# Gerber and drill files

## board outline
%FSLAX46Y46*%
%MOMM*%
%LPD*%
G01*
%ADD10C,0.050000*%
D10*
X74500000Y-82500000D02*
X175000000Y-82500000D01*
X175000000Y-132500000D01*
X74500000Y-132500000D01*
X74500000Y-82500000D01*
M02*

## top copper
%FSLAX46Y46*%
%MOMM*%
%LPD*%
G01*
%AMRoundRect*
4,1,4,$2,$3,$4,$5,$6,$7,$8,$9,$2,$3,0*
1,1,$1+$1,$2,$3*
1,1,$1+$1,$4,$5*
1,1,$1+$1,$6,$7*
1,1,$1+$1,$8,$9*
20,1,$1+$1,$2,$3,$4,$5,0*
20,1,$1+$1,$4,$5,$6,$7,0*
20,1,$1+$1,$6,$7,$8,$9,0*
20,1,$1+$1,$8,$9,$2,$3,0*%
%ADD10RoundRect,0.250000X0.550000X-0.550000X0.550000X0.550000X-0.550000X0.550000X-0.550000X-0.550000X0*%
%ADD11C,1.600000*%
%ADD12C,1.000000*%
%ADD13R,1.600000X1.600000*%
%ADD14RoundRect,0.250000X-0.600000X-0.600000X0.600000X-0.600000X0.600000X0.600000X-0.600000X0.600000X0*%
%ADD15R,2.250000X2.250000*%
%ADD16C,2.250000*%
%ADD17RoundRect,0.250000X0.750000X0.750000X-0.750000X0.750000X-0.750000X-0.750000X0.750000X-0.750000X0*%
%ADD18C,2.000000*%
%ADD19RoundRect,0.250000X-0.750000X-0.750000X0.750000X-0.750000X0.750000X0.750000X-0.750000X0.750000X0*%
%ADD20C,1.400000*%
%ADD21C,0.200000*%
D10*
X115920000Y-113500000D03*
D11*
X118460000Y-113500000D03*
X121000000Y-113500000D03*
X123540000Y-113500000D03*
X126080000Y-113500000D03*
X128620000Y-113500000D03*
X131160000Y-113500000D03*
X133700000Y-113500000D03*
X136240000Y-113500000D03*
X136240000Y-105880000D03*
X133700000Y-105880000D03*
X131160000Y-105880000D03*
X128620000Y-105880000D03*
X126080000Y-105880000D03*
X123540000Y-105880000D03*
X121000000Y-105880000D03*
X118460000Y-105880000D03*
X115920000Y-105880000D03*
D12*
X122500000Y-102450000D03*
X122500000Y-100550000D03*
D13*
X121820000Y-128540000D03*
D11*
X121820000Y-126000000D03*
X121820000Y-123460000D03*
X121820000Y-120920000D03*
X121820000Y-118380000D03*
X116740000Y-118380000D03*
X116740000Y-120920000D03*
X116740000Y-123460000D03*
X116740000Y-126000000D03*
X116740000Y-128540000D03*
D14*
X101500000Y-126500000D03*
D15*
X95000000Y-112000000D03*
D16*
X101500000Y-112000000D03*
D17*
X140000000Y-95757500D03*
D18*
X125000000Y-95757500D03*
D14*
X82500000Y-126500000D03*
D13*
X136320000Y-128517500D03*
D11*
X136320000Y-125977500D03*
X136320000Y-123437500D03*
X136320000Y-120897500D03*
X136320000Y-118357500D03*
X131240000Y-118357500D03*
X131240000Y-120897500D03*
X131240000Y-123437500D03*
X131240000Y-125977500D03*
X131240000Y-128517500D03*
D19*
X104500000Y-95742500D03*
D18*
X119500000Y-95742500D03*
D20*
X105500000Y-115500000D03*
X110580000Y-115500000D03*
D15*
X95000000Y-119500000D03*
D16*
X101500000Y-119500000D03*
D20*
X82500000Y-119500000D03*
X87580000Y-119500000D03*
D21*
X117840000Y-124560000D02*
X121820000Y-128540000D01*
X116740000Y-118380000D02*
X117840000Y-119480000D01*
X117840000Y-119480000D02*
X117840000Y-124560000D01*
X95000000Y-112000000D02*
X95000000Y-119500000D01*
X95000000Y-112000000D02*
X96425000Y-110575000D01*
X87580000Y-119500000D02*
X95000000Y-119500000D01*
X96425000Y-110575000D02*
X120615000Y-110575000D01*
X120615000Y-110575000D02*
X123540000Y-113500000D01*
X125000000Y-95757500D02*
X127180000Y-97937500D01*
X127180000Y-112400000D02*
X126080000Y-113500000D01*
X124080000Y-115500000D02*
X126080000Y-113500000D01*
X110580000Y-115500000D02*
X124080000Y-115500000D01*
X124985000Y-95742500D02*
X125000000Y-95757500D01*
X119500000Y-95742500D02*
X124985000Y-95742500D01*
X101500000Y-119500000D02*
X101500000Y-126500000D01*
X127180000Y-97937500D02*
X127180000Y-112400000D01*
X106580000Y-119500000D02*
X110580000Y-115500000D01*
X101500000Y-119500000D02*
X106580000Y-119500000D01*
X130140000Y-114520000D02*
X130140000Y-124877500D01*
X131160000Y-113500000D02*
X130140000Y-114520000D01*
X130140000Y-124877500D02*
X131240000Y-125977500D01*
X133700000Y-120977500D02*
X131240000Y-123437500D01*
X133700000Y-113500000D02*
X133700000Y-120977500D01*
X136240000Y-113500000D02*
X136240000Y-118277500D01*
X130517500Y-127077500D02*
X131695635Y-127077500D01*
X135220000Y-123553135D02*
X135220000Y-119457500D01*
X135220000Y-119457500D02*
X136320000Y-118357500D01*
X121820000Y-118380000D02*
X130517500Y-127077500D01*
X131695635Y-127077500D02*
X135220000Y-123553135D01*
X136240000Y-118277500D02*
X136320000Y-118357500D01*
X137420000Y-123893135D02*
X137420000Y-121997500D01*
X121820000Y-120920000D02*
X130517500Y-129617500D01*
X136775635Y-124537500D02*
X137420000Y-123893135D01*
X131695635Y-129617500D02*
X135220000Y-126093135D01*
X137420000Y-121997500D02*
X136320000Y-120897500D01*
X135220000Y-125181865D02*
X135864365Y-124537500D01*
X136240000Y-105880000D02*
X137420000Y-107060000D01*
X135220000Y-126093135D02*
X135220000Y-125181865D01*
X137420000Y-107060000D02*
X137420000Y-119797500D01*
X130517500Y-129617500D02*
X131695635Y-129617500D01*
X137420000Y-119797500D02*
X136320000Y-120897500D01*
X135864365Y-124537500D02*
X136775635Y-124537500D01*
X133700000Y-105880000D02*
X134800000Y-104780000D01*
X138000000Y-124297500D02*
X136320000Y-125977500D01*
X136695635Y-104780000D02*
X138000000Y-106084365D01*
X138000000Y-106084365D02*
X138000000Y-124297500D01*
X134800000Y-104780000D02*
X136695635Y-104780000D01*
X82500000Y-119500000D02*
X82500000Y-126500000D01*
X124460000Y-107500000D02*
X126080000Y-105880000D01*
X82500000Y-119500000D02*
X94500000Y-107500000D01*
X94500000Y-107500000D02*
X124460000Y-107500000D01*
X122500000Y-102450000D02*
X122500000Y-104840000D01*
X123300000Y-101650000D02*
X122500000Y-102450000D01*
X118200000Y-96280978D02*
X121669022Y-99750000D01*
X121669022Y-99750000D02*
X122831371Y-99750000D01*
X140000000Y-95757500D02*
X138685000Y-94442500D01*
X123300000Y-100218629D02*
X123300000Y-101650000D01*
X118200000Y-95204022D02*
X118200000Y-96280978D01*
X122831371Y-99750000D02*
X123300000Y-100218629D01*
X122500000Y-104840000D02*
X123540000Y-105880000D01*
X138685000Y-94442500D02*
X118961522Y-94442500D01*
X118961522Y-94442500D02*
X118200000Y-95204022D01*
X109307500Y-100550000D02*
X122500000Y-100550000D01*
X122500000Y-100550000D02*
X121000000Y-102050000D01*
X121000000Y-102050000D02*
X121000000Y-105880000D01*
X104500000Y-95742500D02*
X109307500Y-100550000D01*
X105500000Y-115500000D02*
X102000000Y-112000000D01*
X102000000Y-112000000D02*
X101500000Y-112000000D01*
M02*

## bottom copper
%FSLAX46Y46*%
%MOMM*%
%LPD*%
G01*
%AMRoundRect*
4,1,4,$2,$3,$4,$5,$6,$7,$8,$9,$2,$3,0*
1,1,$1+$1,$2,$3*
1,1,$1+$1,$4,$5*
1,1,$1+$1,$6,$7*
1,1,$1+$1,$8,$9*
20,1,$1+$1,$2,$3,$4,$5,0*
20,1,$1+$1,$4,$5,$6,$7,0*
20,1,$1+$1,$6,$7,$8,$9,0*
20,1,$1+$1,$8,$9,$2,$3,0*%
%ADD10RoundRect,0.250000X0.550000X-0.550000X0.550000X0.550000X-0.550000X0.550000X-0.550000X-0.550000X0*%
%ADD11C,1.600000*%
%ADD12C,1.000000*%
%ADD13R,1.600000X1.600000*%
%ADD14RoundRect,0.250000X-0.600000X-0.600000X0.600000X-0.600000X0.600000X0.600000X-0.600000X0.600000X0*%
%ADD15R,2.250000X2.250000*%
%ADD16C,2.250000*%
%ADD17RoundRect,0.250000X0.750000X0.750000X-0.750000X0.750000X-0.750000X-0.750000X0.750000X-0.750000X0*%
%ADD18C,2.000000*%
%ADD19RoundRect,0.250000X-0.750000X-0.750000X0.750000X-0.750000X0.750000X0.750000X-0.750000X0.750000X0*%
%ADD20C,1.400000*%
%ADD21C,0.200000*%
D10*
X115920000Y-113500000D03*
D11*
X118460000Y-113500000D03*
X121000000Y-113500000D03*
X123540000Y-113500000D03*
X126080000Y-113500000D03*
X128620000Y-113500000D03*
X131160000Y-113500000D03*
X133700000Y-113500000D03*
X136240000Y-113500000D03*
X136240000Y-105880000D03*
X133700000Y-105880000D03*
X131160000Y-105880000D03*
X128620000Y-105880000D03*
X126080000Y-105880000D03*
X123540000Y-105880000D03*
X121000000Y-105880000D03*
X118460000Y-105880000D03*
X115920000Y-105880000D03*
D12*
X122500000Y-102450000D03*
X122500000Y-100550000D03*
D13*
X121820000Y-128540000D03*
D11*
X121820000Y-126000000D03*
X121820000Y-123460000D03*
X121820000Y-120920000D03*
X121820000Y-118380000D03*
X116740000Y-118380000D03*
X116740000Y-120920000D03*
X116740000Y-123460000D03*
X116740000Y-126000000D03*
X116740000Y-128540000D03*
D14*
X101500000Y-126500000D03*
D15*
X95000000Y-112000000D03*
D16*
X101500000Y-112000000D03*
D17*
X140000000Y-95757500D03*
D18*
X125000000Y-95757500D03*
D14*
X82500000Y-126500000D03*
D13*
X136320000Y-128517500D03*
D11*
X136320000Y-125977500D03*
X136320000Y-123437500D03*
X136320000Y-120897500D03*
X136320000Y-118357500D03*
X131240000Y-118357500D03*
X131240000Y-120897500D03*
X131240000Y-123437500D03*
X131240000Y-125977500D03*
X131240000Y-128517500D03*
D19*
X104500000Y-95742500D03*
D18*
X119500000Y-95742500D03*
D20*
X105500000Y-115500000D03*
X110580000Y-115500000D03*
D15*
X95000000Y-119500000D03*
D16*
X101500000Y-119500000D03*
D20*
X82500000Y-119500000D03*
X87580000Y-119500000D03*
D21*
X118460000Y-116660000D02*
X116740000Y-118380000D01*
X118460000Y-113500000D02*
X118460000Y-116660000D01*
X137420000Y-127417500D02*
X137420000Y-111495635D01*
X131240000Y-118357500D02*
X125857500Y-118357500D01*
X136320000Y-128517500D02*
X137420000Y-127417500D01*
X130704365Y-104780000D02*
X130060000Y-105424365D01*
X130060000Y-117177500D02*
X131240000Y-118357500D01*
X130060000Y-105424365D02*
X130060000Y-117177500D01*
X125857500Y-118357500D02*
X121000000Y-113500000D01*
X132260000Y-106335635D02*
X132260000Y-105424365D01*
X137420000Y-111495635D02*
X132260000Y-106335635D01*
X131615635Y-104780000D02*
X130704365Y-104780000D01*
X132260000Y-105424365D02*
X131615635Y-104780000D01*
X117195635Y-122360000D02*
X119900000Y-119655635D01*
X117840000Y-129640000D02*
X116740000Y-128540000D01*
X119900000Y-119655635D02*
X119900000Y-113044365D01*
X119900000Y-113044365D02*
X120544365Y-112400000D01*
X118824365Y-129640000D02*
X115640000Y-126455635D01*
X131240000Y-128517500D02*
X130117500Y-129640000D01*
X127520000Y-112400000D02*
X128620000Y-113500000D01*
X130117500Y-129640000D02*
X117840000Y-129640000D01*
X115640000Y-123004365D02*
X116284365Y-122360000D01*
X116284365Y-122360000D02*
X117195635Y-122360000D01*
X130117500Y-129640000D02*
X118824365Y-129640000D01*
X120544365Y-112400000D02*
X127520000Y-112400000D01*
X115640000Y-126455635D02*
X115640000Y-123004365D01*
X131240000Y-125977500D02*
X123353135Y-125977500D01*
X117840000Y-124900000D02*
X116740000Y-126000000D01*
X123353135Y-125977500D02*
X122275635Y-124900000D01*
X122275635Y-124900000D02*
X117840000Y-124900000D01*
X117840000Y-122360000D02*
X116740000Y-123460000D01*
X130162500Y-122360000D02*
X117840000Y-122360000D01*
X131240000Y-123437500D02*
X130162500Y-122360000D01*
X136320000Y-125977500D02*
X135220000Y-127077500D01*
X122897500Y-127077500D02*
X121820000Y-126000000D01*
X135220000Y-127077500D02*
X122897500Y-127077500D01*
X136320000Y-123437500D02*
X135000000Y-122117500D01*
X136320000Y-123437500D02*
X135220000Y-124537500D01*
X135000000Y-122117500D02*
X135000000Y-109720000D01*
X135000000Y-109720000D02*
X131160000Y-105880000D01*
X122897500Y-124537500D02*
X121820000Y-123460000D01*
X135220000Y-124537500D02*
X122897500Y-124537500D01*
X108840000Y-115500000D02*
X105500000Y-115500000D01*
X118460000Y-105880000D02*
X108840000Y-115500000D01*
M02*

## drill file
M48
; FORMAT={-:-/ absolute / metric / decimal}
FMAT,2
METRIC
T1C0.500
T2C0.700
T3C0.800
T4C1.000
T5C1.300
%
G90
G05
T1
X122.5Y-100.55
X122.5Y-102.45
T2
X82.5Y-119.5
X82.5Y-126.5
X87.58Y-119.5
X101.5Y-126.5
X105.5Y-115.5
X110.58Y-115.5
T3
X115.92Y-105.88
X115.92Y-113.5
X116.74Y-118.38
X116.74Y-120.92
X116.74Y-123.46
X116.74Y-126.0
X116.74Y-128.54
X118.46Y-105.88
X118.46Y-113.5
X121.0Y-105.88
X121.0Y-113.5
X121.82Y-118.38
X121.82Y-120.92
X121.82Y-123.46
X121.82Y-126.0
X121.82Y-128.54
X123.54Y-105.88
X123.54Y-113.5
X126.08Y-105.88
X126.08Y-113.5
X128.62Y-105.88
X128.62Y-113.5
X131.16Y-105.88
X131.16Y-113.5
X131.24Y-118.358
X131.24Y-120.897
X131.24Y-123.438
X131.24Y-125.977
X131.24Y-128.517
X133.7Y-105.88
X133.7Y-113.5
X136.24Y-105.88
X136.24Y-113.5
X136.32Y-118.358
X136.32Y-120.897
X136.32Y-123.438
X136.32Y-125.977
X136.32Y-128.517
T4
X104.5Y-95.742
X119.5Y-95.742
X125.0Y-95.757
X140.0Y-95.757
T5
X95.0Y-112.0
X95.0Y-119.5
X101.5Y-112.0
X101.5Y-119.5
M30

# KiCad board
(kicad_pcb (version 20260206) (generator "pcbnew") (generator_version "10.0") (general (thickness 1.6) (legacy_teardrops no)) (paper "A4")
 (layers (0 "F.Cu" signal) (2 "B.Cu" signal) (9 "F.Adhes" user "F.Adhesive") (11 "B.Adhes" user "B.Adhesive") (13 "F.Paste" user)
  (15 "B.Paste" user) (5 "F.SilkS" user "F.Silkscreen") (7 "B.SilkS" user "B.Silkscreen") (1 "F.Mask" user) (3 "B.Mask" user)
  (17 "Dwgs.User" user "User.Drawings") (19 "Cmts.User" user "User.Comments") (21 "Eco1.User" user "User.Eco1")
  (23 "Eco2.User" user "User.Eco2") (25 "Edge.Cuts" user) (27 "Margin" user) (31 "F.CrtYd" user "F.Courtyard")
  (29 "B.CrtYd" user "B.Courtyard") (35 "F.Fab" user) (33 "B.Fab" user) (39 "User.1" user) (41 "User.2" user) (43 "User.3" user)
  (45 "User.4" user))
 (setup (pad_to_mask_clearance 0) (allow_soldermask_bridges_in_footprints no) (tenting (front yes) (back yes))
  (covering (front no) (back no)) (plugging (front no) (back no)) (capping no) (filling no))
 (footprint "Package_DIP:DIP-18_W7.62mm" (layer "F.Cu") (at 115.92 113.5 90)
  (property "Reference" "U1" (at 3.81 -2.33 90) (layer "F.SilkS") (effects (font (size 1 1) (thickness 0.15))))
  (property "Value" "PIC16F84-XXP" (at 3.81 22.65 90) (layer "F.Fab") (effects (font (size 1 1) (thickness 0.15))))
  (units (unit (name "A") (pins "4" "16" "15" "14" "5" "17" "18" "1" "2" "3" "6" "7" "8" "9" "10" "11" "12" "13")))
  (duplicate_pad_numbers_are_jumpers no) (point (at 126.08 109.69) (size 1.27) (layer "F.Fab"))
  (pad "1" thru_hole roundrect (at 0 0 90) (size 1.6 1.6) (drill 0.8) (layers "*.Cu" "*.Mask") (remove_unused_layers no)
   (roundrect_rratio 0.15625) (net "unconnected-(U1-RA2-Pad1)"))
  (pad "2" thru_hole circle (at 0 2.54 90) (size 1.6 1.6) (drill 0.8) (layers "*.Cu" "*.Mask") (remove_unused_layers no)
   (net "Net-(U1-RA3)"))
  (pad "3" thru_hole circle (at 0 5.08 90) (size 1.6 1.6) (drill 0.8) (layers "*.Cu" "*.Mask") (remove_unused_layers no)
   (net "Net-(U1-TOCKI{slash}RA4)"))
  (pad "4" thru_hole circle (at 0 7.62 90) (size 1.6 1.6) (drill 0.8) (layers "*.Cu" "*.Mask") (remove_unused_layers no)
   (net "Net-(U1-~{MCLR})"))
  (pad "5" thru_hole circle (at 0 10.16 90) (size 1.6 1.6) (drill 0.8) (layers "*.Cu" "*.Mask") (remove_unused_layers no) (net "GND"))
  (pad "6" thru_hole circle (at 0 12.7 90) (size 1.6 1.6) (drill 0.8) (layers "*.Cu" "*.Mask") (remove_unused_layers no)
   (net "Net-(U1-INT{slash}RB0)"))
  (pad "7" thru_hole circle (at 0 15.24 90) (size 1.6 1.6) (drill 0.8) (layers "*.Cu" "*.Mask") (remove_unused_layers no)
   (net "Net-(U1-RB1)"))
  (pad "8" thru_hole circle (at 0 17.78 90) (size 1.6 1.6) (drill 0.8) (layers "*.Cu" "*.Mask") (remove_unused_layers no)
   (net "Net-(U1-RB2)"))
  (pad "9" thru_hole circle (at 0 20.32 90) (size 1.6 1.6) (drill 0.8) (layers "*.Cu" "*.Mask") (remove_unused_layers no)
   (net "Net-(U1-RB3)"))
  (pad "10" thru_hole circle (at 7.62 20.32 90) (size 1.6 1.6) (drill 0.8) (layers "*.Cu" "*.Mask") (remove_unused_layers no)
   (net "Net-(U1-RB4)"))
  (pad "11" thru_hole circle (at 7.62 17.78 90) (size 1.6 1.6) (drill 0.8) (layers "*.Cu" "*.Mask") (remove_unused_layers no)
   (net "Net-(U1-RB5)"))
  (pad "12" thru_hole circle (at 7.62 15.24 90) (size 1.6 1.6) (drill 0.8) (layers "*.Cu" "*.Mask") (remove_unused_layers no)
   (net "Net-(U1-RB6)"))
  (pad "13" thru_hole circle (at 7.62 12.7 90) (size 1.6 1.6) (drill 0.8) (layers "*.Cu" "*.Mask") (remove_unused_layers no)
   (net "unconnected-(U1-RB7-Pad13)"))
  (pad "14" thru_hole circle (at 7.62 10.16 90) (size 1.6 1.6) (drill 0.8) (layers "*.Cu" "*.Mask") (remove_unused_layers no) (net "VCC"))
  (pad "15" thru_hole circle (at 7.62 7.62 90) (size 1.6 1.6) (drill 0.8) (layers "*.Cu" "*.Mask") (remove_unused_layers no)
   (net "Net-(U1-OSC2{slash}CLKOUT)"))
  (pad "16" thru_hole circle (at 7.62 5.08 90) (size 1.6 1.6) (drill 0.8) (layers "*.Cu" "*.Mask") (remove_unused_layers no)
   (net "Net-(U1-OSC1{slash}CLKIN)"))
  (pad "17" thru_hole circle (at 7.62 2.54 90) (size 1.6 1.6) (drill 0.8) (layers "*.Cu" "*.Mask") (remove_unused_layers no)
   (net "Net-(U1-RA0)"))
  (pad "18" thru_hole circle (at 7.62 0 90) (size 1.6 1.6) (drill 0.8) (layers "*.Cu" "*.Mask") (remove_unused_layers no)
   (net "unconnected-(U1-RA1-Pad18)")))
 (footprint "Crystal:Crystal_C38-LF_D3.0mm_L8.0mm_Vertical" (layer "F.Cu") (at 122.5 102.45 90)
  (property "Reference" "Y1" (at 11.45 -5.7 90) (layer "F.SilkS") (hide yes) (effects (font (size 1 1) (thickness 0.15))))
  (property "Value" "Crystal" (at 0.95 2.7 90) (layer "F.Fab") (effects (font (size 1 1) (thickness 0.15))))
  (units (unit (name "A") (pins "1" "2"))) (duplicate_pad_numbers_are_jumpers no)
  (pad "1" thru_hole circle (at 0 0 90) (size 1 1) (drill 0.5) (layers "*.Cu" "*.Mask") (remove_unused_layers no)
   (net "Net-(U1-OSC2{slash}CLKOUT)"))
  (pad "2" thru_hole circle (at 1.9 0 90) (size 1 1) (drill 0.5) (layers "*.Cu" "*.Mask") (remove_unused_layers no)
   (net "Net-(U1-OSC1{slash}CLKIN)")))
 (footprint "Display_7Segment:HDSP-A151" (layer "F.Cu") (at 121.82 128.54 180)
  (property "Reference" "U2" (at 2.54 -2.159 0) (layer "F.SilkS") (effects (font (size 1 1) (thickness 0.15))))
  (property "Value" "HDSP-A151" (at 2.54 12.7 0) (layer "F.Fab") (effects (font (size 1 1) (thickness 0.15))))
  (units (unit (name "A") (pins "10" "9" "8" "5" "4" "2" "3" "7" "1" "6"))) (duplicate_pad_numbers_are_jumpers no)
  (pad "1" thru_hole rect (at 0 0 180) (size 1.6 1.6) (drill 0.8) (layers "*.Cu" "*.Mask") (remove_unused_layers no) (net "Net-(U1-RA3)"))
  (pad "2" thru_hole circle (at 0 2.54 180) (size 1.6 1.6) (drill 0.8) (layers "*.Cu" "*.Mask") (remove_unused_layers no)
   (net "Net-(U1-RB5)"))
  (pad "3" thru_hole circle (at 0 5.08 180) (size 1.6 1.6) (drill 0.8) (layers "*.Cu" "*.Mask") (remove_unused_layers no)
   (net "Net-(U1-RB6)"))
  (pad "4" thru_hole circle (at 0 7.62 180) (size 1.6 1.6) (drill 0.8) (layers "*.Cu" "*.Mask") (remove_unused_layers no)
   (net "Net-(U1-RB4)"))
  (pad "5" thru_hole circle (at 0 10.16 180) (size 1.6 1.6) (drill 0.8) (layers "*.Cu" "*.Mask") (remove_unused_layers no)
   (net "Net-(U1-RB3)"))
  (pad "6" thru_hole circle (at 5.08 10.16 180) (size 1.6 1.6) (drill 0.8) (layers "*.Cu" "*.Mask") (remove_unused_layers no)
   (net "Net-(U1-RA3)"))
  (pad "7" thru_hole circle (at 5.08 7.62 180) (size 1.6 1.6) (drill 0.8) (layers "*.Cu" "*.Mask") (remove_unused_layers no)
   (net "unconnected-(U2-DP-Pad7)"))
  (pad "8" thru_hole circle (at 5.08 5.08 180) (size 1.6 1.6) (drill 0.8) (layers "*.Cu" "*.Mask") (remove_unused_layers no)
   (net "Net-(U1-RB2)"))
  (pad "9" thru_hole circle (at 5.08 2.54 180) (size 1.6 1.6) (drill 0.8) (layers "*.Cu" "*.Mask") (remove_unused_layers no)
   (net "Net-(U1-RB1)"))
  (pad "10" thru_hole circle (at 5.08 0 180) (size 1.6 1.6) (drill 0.8) (layers "*.Cu" "*.Mask") (remove_unused_layers no)
   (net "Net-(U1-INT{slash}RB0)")))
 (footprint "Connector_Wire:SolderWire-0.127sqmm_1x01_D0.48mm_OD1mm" (layer "F.Cu") (at 101.5 126.5)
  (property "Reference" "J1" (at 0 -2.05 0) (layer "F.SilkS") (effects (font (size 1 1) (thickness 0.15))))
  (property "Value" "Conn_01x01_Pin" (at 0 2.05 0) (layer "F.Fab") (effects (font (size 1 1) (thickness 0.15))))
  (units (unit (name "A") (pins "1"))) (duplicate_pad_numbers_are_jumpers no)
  (pad "1" thru_hole roundrect (at 0 0) (size 1.7 1.7) (drill 0.7) (layers "*.Cu" "*.Mask") (remove_unused_layers no)
   (roundrect_rratio 0.147059) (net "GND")))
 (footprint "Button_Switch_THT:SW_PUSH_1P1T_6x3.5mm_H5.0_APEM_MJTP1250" (layer "F.Cu") (at 95 112)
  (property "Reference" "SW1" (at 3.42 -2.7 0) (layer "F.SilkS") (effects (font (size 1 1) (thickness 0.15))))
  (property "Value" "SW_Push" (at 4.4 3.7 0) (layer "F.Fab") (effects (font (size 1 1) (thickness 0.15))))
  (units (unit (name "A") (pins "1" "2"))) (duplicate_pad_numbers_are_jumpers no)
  (pad "1" thru_hole rect (at 0 0 90) (size 2.25 2.25) (drill 1.3) (layers "*.Cu" "*.Mask") (remove_unused_layers no)
   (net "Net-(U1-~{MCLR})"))
  (pad "2" thru_hole circle (at 6.5 0 90) (size 2.25 2.25) (drill 1.3) (layers "*.Cu" "*.Mask") (remove_unused_layers no)
   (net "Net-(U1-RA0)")))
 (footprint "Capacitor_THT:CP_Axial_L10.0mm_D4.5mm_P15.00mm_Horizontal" (layer "F.Cu") (at 140 95.7575 180)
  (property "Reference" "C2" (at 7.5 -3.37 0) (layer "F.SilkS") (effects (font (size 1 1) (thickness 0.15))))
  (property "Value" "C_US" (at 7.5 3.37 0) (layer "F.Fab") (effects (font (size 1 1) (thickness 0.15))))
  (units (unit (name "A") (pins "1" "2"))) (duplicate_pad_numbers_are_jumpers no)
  (pad "1" thru_hole roundrect (at 0 0 180) (size 2 2) (drill 1) (layers "*.Cu" "*.Mask") (remove_unused_layers no) (roundrect_rratio 0.125)
   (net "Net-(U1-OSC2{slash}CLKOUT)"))
  (pad "2" thru_hole circle (at 15 0 180) (size 2 2) (drill 1) (layers "*.Cu" "*.Mask") (remove_unused_layers no) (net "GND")))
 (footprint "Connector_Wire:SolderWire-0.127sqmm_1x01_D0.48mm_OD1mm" (layer "F.Cu") (at 82.5 126.5)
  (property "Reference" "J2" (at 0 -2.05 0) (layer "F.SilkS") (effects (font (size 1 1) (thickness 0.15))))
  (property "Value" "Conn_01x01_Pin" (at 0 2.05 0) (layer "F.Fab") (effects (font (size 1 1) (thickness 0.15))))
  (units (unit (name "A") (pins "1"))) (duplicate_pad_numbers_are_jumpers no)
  (pad "1" thru_hole roundrect (at 0 0) (size 1.7 1.7) (drill 0.7) (layers "*.Cu" "*.Mask") (remove_unused_layers no)
   (roundrect_rratio 0.147059) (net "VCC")))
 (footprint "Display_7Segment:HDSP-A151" (layer "F.Cu") (at 136.32 128.5175 180)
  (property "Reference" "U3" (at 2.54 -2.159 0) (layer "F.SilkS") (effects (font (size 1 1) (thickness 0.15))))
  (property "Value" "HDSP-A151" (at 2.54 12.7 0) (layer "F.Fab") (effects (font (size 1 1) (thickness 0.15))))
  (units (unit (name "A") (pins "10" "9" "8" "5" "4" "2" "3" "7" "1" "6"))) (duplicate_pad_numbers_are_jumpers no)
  (pad "1" thru_hole rect (at 0 0 180) (size 1.6 1.6) (drill 0.8) (layers "*.Cu" "*.Mask") (remove_unused_layers no)
   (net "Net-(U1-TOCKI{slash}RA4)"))
  (pad "2" thru_hole circle (at 0 2.54 180) (size 1.6 1.6) (drill 0.8) (layers "*.Cu" "*.Mask") (remove_unused_layers no)
   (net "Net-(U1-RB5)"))
  (pad "3" thru_hole circle (at 0 5.08 180) (size 1.6 1.6) (drill 0.8) (layers "*.Cu" "*.Mask") (remove_unused_layers no)
   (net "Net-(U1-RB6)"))
  (pad "4" thru_hole circle (at 0 7.62 180) (size 1.6 1.6) (drill 0.8) (layers "*.Cu" "*.Mask") (remove_unused_layers no)
   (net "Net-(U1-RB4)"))
  (pad "5" thru_hole circle (at 0 10.16 180) (size 1.6 1.6) (drill 0.8) (layers "*.Cu" "*.Mask") (remove_unused_layers no)
   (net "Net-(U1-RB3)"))
  (pad "6" thru_hole circle (at 5.08 10.16 180) (size 1.6 1.6) (drill 0.8) (layers "*.Cu" "*.Mask") (remove_unused_layers no)
   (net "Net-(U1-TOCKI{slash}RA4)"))
  (pad "7" thru_hole circle (at 5.08 7.62 180) (size 1.6 1.6) (drill 0.8) (layers "*.Cu" "*.Mask") (remove_unused_layers no)
   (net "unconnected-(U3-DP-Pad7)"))
  (pad "8" thru_hole circle (at 5.08 5.08 180) (size 1.6 1.6) (drill 0.8) (layers "*.Cu" "*.Mask") (remove_unused_layers no)
   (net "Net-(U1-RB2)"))
  (pad "9" thru_hole circle (at 5.08 2.54 180) (size 1.6 1.6) (drill 0.8) (layers "*.Cu" "*.Mask") (remove_unused_layers no)
   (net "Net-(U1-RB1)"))
  (pad "10" thru_hole circle (at 5.08 0 180) (size 1.6 1.6) (drill 0.8) (layers "*.Cu" "*.Mask") (remove_unused_layers no)
   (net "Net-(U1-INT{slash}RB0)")))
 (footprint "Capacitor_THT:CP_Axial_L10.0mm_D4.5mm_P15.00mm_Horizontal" (layer "F.Cu") (at 104.5 95.7425)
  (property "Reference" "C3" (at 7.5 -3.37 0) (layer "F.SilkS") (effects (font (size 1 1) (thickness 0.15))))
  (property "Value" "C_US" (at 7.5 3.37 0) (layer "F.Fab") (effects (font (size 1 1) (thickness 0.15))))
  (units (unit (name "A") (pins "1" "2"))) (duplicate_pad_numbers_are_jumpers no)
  (pad "1" thru_hole roundrect (at 0 0) (size 2 2) (drill 1) (layers "*.Cu" "*.Mask") (remove_unused_layers no) (roundrect_rratio 0.125)
   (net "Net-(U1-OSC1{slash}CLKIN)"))
  (pad "2" thru_hole circle (at 15 0) (size 2 2) (drill 1) (layers "*.Cu" "*.Mask") (remove_unused_layers no) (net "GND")))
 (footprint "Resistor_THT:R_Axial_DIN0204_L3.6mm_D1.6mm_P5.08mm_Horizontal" (layer "F.Cu") (at 105.5 115.5)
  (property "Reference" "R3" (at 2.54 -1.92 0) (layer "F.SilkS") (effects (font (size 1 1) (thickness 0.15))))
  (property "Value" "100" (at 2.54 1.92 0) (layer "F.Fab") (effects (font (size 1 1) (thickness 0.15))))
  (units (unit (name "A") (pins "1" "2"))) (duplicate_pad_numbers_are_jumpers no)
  (pad "1" thru_hole circle (at 0 0) (size 1.4 1.4) (drill 0.7) (layers "*.Cu" "*.Mask") (remove_unused_layers no) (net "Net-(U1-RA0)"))
  (pad "2" thru_hole circle (at 5.08 0) (size 1.4 1.4) (drill 0.7) (layers "*.Cu" "*.Mask") (remove_unused_layers no) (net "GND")))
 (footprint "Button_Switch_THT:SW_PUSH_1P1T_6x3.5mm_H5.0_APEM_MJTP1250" (layer "F.Cu") (at 95 119.5)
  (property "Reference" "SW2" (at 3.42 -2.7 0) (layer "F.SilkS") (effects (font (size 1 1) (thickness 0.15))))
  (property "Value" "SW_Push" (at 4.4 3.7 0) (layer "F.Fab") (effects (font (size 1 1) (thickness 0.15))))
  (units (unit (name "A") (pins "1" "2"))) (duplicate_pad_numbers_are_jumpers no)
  (pad "1" thru_hole rect (at 0 0 90) (size 2.25 2.25) (drill 1.3) (layers "*.Cu" "*.Mask") (remove_unused_layers no)
   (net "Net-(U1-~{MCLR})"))
  (pad "2" thru_hole circle (at 6.5 0 90) (size 2.25 2.25) (drill 1.3) (layers "*.Cu" "*.Mask") (remove_unused_layers no) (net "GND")))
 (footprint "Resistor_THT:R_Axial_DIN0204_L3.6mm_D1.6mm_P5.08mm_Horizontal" (layer "F.Cu") (at 82.5 119.5)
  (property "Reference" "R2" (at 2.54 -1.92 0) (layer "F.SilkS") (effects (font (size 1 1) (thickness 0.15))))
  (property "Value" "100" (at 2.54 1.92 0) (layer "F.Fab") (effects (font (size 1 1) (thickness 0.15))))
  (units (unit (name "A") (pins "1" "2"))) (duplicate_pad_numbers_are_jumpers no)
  (pad "1" thru_hole circle (at 0 0) (size 1.4 1.4) (drill 0.7) (layers "*.Cu" "*.Mask") (remove_unused_layers no) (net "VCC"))
  (pad "2" thru_hole circle (at 5.08 0) (size 1.4 1.4) (drill 0.7) (layers "*.Cu" "*.Mask") (remove_unused_layers no)
   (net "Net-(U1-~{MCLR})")))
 (gr_rect (start 74.5 82.5) (end 175 132.5) (stroke (width 0.05) (type default)) (fill no) (layer "Edge.Cuts"))
 (segment (start 117.84 124.56) (end 121.82 128.54) (width 0.2) (layer "F.Cu") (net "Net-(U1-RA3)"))
 (segment (start 116.74 118.38) (end 117.84 119.48) (width 0.2) (layer "F.Cu") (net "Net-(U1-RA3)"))
 (segment (start 117.84 119.48) (end 117.84 124.56) (width 0.2) (layer "F.Cu") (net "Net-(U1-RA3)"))
 (segment (start 118.46 116.66) (end 116.74 118.38) (width 0.2) (layer "B.Cu") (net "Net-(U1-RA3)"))
 (segment (start 118.46 113.5) (end 118.46 116.66) (width 0.2) (layer "B.Cu") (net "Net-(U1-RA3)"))
 (segment (start 137.42 127.4175) (end 137.42 111.495635) (width 0.2) (layer "B.Cu") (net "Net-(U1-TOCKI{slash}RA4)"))
 (segment (start 131.24 118.3575) (end 125.8575 118.3575) (width 0.2) (layer "B.Cu") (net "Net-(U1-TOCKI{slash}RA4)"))
 (segment (start 136.32 128.5175) (end 137.42 127.4175) (width 0.2) (layer "B.Cu") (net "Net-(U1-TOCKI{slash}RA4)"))
 (segment (start 130.704365 104.78) (end 130.06 105.424365) (width 0.2) (layer "B.Cu") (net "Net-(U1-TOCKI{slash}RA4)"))
 (segment (start 130.06 117.1775) (end 131.24 118.3575) (width 0.2) (layer "B.Cu") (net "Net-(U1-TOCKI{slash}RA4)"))
 (segment (start 130.06 105.424365) (end 130.06 117.1775) (width 0.2) (layer "B.Cu") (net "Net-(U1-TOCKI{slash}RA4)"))
 (segment (start 125.8575 118.3575) (end 121 113.5) (width 0.2) (layer "B.Cu") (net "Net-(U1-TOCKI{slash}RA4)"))
 (segment (start 132.26 106.335635) (end 132.26 105.424365) (width 0.2) (layer "B.Cu") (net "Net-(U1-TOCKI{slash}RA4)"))
 (segment (start 137.42 111.495635) (end 132.26 106.335635) (width 0.2) (layer "B.Cu") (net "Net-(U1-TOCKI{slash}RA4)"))
 (segment (start 131.615635 104.78) (end 130.704365 104.78) (width 0.2) (layer "B.Cu") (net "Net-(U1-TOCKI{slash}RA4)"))
 (segment (start 132.26 105.424365) (end 131.615635 104.78) (width 0.2) (layer "B.Cu") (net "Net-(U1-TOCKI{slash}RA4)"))
 (segment (start 95 112) (end 95 119.5) (width 0.2) (layer "F.Cu") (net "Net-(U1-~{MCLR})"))
 (segment (start 95 112) (end 96.425 110.575) (width 0.2) (layer "F.Cu") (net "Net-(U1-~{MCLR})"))
 (segment (start 87.58 119.5) (end 95 119.5) (width 0.2) (layer "F.Cu") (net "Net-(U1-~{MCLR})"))
 (segment (start 96.425 110.575) (end 120.615 110.575) (width 0.2) (layer "F.Cu") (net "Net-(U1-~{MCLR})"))
 (segment (start 120.615 110.575) (end 123.54 113.5) (width 0.2) (layer "F.Cu") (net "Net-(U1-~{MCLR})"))
 (segment (start 125 95.7575) (end 127.18 97.9375) (width 0.2) (layer "F.Cu") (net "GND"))
 (segment (start 127.18 112.4) (end 126.08 113.5) (width 0.2) (layer "F.Cu") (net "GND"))
 (segment (start 124.08 115.5) (end 126.08 113.5) (width 0.2) (layer "F.Cu") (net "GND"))
 (segment (start 110.58 115.5) (end 124.08 115.5) (width 0.2) (layer "F.Cu") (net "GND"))
 (segment (start 124.985 95.7425) (end 125 95.7575) (width 0.2) (layer "F.Cu") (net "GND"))
 (segment (start 119.5 95.7425) (end 124.985 95.7425) (width 0.2) (layer "F.Cu") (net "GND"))
 (segment (start 101.5 119.5) (end 101.5 126.5) (width 0.2) (layer "F.Cu") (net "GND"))
 (segment (start 127.18 97.9375) (end 127.18 112.4) (width 0.2) (layer "F.Cu") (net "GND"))
 (segment (start 106.58 119.5) (end 110.58 115.5) (width 0.2) (layer "F.Cu") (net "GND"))
 (segment (start 101.5 119.5) (end 106.58 119.5) (width 0.2) (layer "F.Cu") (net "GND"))
 (segment (start 117.195635 122.36) (end 119.9 119.655635) (width 0.2) (layer "B.Cu") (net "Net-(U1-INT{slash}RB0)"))
 (segment (start 117.84 129.64) (end 116.74 128.54) (width 0.2) (layer "B.Cu") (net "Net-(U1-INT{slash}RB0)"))
 (segment (start 119.9 119.655635) (end 119.9 113.044365) (width 0.2) (layer "B.Cu") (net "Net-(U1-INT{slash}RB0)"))
 (segment (start 119.9 113.044365) (end 120.544365 112.4) (width 0.2) (layer "B.Cu") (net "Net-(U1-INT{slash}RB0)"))
 (segment (start 118.824365 129.64) (end 115.64 126.455635) (width 0.2) (layer "B.Cu") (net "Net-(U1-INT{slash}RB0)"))
 (segment (start 131.24 128.5175) (end 130.1175 129.64) (width 0.2) (layer "B.Cu") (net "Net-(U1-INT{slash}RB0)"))
 (segment (start 127.52 112.4) (end 128.62 113.5) (width 0.2) (layer "B.Cu") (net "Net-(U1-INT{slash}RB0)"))
 (segment (start 130.1175 129.64) (end 117.84 129.64) (width 0.2) (layer "B.Cu") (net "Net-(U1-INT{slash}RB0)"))
 (segment (start 115.64 123.004365) (end 116.284365 122.36) (width 0.2) (layer "B.Cu") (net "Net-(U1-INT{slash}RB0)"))
 (segment (start 116.284365 122.36) (end 117.195635 122.36) (width 0.2) (layer "B.Cu") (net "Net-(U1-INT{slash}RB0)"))
 (segment (start 130.1175 129.64) (end 118.824365 129.64) (width 0.2) (layer "B.Cu") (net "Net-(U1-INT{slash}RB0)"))
 (segment (start 120.544365 112.4) (end 127.52 112.4) (width 0.2) (layer "B.Cu") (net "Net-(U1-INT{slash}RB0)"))
 (segment (start 115.64 126.455635) (end 115.64 123.004365) (width 0.2) (layer "B.Cu") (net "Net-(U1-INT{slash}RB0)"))
 (segment (start 130.14 114.52) (end 130.14 124.8775) (width 0.2) (layer "F.Cu") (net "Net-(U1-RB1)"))
 (segment (start 131.16 113.5) (end 130.14 114.52) (width 0.2) (layer "F.Cu") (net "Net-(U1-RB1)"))
 (segment (start 130.14 124.8775) (end 131.24 125.9775) (width 0.2) (layer "F.Cu") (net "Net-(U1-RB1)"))
 (segment (start 131.24 125.9775) (end 123.353135 125.9775) (width 0.2) (layer "B.Cu") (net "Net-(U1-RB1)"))
 (segment (start 117.84 124.9) (end 116.74 126) (width 0.2) (layer "B.Cu") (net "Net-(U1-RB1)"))
 (segment (start 123.353135 125.9775) (end 122.275635 124.9) (width 0.2) (layer "B.Cu") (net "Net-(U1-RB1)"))
 (segment (start 122.275635 124.9) (end 117.84 124.9) (width 0.2) (layer "B.Cu") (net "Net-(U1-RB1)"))
 (segment (start 133.7 120.9775) (end 131.24 123.4375) (width 0.2) (layer "F.Cu") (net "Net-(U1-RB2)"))
 (segment (start 133.7 113.5) (end 133.7 120.9775) (width 0.2) (layer "F.Cu") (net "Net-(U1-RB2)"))
 (segment (start 117.84 122.36) (end 116.74 123.46) (width 0.2) (layer "B.Cu") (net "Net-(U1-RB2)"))
 (segment (start 130.1625 122.36) (end 117.84 122.36) (width 0.2) (layer "B.Cu") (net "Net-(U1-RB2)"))
 (segment (start 131.24 123.4375) (end 130.1625 122.36) (width 0.2) (layer "B.Cu") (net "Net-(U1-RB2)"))
 (segment (start 136.24 113.5) (end 136.24 118.2775) (width 0.2) (layer "F.Cu") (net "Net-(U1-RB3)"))
 (segment (start 130.5175 127.0775) (end 131.695635 127.0775) (width 0.2) (layer "F.Cu") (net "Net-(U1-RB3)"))
 (segment (start 135.22 123.553135) (end 135.22 119.4575) (width 0.2) (layer "F.Cu") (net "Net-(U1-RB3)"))
 (segment (start 135.22 119.4575) (end 136.32 118.3575) (width 0.2) (layer "F.Cu") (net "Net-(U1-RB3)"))
 (segment (start 121.82 118.38) (end 130.5175 127.0775) (width 0.2) (layer "F.Cu") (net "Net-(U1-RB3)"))
 (segment (start 131.695635 127.0775) (end 135.22 123.553135) (width 0.2) (layer "F.Cu") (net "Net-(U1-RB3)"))
 (segment (start 136.24 118.2775) (end 136.32 118.3575) (width 0.2) (layer "F.Cu") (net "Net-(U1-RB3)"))
 (segment (start 137.42 123.893135) (end 137.42 121.9975) (width 0.2) (layer "F.Cu") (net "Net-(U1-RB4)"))
 (segment (start 121.82 120.92) (end 130.5175 129.6175) (width 0.2) (layer "F.Cu") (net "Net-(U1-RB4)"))
 (segment (start 136.775635 124.5375) (end 137.42 123.893135) (width 0.2) (layer "F.Cu") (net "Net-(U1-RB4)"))
 (segment (start 131.695635 129.6175) (end 135.22 126.093135) (width 0.2) (layer "F.Cu") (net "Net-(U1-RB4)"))
 (segment (start 137.42 121.9975) (end 136.32 120.8975) (width 0.2) (layer "F.Cu") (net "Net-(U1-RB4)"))
 (segment (start 135.22 125.181865) (end 135.864365 124.5375) (width 0.2) (layer "F.Cu") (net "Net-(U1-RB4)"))
 (segment (start 136.24 105.88) (end 137.42 107.06) (width 0.2) (layer "F.Cu") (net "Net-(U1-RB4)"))
 (segment (start 135.22 126.093135) (end 135.22 125.181865) (width 0.2) (layer "F.Cu") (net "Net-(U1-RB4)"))
 (segment (start 137.42 107.06) (end 137.42 119.7975) (width 0.2) (layer "F.Cu") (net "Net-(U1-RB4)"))
 (segment (start 130.5175 129.6175) (end 131.695635 129.6175) (width 0.2) (layer "F.Cu") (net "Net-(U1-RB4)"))
 (segment (start 137.42 119.7975) (end 136.32 120.8975) (width 0.2) (layer "F.Cu") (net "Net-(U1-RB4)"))
 (segment (start 135.864365 124.5375) (end 136.775635 124.5375) (width 0.2) (layer "F.Cu") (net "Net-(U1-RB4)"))
 (segment (start 133.7 105.88) (end 134.8 104.78) (width 0.2) (layer "F.Cu") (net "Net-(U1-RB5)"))
 (segment (start 138 124.2975) (end 136.32 125.9775) (width 0.2) (layer "F.Cu") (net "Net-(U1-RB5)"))
 (segment (start 136.695635 104.78) (end 138 106.084365) (width 0.2) (layer "F.Cu") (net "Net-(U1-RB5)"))
 (segment (start 138 106.084365) (end 138 124.2975) (width 0.2) (layer "F.Cu") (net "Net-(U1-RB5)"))
 (segment (start 134.8 104.78) (end 136.695635 104.78) (width 0.2) (layer "F.Cu") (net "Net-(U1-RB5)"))
 (segment (start 136.32 125.9775) (end 135.22 127.0775) (width 0.2) (layer "B.Cu") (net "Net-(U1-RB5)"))
 (segment (start 122.8975 127.0775) (end 121.82 126) (width 0.2) (layer "B.Cu") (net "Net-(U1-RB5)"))
 (segment (start 135.22 127.0775) (end 122.8975 127.0775) (width 0.2) (layer "B.Cu") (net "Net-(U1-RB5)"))
 (segment (start 136.32 123.4375) (end 135 122.1175) (width 0.2) (layer "B.Cu") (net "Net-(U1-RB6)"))
 (segment (start 136.32 123.4375) (end 135.22 124.5375) (width 0.2) (layer "B.Cu") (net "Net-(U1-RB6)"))
 (segment (start 135 122.1175) (end 135 109.72) (width 0.2) (layer "B.Cu") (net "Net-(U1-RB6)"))
 (segment (start 135 109.72) (end 131.16 105.88) (width 0.2) (layer "B.Cu") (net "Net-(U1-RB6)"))
 (segment (start 122.8975 124.5375) (end 121.82 123.46) (width 0.2) (layer "B.Cu") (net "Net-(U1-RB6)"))
 (segment (start 135.22 124.5375) (end 122.8975 124.5375) (width 0.2) (layer "B.Cu") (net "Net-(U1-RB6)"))
 (segment (start 82.5 119.5) (end 82.5 126.5) (width 0.2) (layer "F.Cu") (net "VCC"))
 (segment (start 124.46 107.5) (end 126.08 105.88) (width 0.2) (layer "F.Cu") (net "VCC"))
 (segment (start 82.5 119.5) (end 94.5 107.5) (width 0.2) (layer "F.Cu") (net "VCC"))
 (segment (start 94.5 107.5) (end 124.46 107.5) (width 0.2) (layer "F.Cu") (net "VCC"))
 (segment (start 122.5 102.45) (end 122.5 104.84) (width 0.2) (layer "F.Cu") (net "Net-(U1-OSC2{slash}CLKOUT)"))
 (segment (start 123.3 101.65) (end 122.5 102.45) (width 0.2) (layer "F.Cu") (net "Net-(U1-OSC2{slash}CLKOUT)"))
 (segment (start 118.2 96.280978) (end 121.669022 99.75) (width 0.2) (layer "F.Cu") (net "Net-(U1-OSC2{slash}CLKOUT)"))
 (segment (start 121.669022 99.75) (end 122.831371 99.75) (width 0.2) (layer "F.Cu") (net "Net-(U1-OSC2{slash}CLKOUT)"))
 (segment (start 140 95.7575) (end 138.685 94.4425) (width 0.2) (layer "F.Cu") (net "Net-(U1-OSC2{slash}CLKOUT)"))
 (segment (start 123.3 100.218629) (end 123.3 101.65) (width 0.2) (layer "F.Cu") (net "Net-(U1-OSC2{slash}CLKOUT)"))
 (segment (start 118.2 95.204022) (end 118.2 96.280978) (width 0.2) (layer "F.Cu") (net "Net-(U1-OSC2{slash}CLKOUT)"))
 (segment (start 122.831371 99.75) (end 123.3 100.218629) (width 0.2) (layer "F.Cu") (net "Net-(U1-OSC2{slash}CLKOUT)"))
 (segment (start 122.5 104.84) (end 123.54 105.88) (width 0.2) (layer "F.Cu") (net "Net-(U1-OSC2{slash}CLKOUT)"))
 (segment (start 138.685 94.4425) (end 118.961522 94.4425) (width 0.2) (layer "F.Cu") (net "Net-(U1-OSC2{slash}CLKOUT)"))
 (segment (start 118.961522 94.4425) (end 118.2 95.204022) (width 0.2) (layer "F.Cu") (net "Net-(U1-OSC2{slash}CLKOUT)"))
 (segment (start 109.3075 100.55) (end 122.5 100.55) (width 0.2) (layer "F.Cu") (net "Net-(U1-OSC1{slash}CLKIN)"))
 (segment (start 122.5 100.55) (end 121 102.05) (width 0.2) (layer "F.Cu") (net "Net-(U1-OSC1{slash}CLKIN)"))
 (segment (start 121 102.05) (end 121 105.88) (width 0.2) (layer "F.Cu") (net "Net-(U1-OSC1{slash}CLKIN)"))
 (segment (start 104.5 95.7425) (end 109.3075 100.55) (width 0.2) (layer "F.Cu") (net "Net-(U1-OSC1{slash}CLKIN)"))
 (segment (start 105.5 115.5) (end 102 112) (width 0.2) (layer "F.Cu") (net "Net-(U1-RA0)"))
 (segment (start 102 112) (end 101.5 112) (width 0.2) (layer "F.Cu") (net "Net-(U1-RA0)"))
 (segment (start 108.84 115.5) (end 105.5 115.5) (width 0.2) (layer "B.Cu") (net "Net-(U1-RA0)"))
 (segment (start 118.46 105.88) (end 108.84 115.5) (width 0.2) (layer "B.Cu") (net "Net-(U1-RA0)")))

